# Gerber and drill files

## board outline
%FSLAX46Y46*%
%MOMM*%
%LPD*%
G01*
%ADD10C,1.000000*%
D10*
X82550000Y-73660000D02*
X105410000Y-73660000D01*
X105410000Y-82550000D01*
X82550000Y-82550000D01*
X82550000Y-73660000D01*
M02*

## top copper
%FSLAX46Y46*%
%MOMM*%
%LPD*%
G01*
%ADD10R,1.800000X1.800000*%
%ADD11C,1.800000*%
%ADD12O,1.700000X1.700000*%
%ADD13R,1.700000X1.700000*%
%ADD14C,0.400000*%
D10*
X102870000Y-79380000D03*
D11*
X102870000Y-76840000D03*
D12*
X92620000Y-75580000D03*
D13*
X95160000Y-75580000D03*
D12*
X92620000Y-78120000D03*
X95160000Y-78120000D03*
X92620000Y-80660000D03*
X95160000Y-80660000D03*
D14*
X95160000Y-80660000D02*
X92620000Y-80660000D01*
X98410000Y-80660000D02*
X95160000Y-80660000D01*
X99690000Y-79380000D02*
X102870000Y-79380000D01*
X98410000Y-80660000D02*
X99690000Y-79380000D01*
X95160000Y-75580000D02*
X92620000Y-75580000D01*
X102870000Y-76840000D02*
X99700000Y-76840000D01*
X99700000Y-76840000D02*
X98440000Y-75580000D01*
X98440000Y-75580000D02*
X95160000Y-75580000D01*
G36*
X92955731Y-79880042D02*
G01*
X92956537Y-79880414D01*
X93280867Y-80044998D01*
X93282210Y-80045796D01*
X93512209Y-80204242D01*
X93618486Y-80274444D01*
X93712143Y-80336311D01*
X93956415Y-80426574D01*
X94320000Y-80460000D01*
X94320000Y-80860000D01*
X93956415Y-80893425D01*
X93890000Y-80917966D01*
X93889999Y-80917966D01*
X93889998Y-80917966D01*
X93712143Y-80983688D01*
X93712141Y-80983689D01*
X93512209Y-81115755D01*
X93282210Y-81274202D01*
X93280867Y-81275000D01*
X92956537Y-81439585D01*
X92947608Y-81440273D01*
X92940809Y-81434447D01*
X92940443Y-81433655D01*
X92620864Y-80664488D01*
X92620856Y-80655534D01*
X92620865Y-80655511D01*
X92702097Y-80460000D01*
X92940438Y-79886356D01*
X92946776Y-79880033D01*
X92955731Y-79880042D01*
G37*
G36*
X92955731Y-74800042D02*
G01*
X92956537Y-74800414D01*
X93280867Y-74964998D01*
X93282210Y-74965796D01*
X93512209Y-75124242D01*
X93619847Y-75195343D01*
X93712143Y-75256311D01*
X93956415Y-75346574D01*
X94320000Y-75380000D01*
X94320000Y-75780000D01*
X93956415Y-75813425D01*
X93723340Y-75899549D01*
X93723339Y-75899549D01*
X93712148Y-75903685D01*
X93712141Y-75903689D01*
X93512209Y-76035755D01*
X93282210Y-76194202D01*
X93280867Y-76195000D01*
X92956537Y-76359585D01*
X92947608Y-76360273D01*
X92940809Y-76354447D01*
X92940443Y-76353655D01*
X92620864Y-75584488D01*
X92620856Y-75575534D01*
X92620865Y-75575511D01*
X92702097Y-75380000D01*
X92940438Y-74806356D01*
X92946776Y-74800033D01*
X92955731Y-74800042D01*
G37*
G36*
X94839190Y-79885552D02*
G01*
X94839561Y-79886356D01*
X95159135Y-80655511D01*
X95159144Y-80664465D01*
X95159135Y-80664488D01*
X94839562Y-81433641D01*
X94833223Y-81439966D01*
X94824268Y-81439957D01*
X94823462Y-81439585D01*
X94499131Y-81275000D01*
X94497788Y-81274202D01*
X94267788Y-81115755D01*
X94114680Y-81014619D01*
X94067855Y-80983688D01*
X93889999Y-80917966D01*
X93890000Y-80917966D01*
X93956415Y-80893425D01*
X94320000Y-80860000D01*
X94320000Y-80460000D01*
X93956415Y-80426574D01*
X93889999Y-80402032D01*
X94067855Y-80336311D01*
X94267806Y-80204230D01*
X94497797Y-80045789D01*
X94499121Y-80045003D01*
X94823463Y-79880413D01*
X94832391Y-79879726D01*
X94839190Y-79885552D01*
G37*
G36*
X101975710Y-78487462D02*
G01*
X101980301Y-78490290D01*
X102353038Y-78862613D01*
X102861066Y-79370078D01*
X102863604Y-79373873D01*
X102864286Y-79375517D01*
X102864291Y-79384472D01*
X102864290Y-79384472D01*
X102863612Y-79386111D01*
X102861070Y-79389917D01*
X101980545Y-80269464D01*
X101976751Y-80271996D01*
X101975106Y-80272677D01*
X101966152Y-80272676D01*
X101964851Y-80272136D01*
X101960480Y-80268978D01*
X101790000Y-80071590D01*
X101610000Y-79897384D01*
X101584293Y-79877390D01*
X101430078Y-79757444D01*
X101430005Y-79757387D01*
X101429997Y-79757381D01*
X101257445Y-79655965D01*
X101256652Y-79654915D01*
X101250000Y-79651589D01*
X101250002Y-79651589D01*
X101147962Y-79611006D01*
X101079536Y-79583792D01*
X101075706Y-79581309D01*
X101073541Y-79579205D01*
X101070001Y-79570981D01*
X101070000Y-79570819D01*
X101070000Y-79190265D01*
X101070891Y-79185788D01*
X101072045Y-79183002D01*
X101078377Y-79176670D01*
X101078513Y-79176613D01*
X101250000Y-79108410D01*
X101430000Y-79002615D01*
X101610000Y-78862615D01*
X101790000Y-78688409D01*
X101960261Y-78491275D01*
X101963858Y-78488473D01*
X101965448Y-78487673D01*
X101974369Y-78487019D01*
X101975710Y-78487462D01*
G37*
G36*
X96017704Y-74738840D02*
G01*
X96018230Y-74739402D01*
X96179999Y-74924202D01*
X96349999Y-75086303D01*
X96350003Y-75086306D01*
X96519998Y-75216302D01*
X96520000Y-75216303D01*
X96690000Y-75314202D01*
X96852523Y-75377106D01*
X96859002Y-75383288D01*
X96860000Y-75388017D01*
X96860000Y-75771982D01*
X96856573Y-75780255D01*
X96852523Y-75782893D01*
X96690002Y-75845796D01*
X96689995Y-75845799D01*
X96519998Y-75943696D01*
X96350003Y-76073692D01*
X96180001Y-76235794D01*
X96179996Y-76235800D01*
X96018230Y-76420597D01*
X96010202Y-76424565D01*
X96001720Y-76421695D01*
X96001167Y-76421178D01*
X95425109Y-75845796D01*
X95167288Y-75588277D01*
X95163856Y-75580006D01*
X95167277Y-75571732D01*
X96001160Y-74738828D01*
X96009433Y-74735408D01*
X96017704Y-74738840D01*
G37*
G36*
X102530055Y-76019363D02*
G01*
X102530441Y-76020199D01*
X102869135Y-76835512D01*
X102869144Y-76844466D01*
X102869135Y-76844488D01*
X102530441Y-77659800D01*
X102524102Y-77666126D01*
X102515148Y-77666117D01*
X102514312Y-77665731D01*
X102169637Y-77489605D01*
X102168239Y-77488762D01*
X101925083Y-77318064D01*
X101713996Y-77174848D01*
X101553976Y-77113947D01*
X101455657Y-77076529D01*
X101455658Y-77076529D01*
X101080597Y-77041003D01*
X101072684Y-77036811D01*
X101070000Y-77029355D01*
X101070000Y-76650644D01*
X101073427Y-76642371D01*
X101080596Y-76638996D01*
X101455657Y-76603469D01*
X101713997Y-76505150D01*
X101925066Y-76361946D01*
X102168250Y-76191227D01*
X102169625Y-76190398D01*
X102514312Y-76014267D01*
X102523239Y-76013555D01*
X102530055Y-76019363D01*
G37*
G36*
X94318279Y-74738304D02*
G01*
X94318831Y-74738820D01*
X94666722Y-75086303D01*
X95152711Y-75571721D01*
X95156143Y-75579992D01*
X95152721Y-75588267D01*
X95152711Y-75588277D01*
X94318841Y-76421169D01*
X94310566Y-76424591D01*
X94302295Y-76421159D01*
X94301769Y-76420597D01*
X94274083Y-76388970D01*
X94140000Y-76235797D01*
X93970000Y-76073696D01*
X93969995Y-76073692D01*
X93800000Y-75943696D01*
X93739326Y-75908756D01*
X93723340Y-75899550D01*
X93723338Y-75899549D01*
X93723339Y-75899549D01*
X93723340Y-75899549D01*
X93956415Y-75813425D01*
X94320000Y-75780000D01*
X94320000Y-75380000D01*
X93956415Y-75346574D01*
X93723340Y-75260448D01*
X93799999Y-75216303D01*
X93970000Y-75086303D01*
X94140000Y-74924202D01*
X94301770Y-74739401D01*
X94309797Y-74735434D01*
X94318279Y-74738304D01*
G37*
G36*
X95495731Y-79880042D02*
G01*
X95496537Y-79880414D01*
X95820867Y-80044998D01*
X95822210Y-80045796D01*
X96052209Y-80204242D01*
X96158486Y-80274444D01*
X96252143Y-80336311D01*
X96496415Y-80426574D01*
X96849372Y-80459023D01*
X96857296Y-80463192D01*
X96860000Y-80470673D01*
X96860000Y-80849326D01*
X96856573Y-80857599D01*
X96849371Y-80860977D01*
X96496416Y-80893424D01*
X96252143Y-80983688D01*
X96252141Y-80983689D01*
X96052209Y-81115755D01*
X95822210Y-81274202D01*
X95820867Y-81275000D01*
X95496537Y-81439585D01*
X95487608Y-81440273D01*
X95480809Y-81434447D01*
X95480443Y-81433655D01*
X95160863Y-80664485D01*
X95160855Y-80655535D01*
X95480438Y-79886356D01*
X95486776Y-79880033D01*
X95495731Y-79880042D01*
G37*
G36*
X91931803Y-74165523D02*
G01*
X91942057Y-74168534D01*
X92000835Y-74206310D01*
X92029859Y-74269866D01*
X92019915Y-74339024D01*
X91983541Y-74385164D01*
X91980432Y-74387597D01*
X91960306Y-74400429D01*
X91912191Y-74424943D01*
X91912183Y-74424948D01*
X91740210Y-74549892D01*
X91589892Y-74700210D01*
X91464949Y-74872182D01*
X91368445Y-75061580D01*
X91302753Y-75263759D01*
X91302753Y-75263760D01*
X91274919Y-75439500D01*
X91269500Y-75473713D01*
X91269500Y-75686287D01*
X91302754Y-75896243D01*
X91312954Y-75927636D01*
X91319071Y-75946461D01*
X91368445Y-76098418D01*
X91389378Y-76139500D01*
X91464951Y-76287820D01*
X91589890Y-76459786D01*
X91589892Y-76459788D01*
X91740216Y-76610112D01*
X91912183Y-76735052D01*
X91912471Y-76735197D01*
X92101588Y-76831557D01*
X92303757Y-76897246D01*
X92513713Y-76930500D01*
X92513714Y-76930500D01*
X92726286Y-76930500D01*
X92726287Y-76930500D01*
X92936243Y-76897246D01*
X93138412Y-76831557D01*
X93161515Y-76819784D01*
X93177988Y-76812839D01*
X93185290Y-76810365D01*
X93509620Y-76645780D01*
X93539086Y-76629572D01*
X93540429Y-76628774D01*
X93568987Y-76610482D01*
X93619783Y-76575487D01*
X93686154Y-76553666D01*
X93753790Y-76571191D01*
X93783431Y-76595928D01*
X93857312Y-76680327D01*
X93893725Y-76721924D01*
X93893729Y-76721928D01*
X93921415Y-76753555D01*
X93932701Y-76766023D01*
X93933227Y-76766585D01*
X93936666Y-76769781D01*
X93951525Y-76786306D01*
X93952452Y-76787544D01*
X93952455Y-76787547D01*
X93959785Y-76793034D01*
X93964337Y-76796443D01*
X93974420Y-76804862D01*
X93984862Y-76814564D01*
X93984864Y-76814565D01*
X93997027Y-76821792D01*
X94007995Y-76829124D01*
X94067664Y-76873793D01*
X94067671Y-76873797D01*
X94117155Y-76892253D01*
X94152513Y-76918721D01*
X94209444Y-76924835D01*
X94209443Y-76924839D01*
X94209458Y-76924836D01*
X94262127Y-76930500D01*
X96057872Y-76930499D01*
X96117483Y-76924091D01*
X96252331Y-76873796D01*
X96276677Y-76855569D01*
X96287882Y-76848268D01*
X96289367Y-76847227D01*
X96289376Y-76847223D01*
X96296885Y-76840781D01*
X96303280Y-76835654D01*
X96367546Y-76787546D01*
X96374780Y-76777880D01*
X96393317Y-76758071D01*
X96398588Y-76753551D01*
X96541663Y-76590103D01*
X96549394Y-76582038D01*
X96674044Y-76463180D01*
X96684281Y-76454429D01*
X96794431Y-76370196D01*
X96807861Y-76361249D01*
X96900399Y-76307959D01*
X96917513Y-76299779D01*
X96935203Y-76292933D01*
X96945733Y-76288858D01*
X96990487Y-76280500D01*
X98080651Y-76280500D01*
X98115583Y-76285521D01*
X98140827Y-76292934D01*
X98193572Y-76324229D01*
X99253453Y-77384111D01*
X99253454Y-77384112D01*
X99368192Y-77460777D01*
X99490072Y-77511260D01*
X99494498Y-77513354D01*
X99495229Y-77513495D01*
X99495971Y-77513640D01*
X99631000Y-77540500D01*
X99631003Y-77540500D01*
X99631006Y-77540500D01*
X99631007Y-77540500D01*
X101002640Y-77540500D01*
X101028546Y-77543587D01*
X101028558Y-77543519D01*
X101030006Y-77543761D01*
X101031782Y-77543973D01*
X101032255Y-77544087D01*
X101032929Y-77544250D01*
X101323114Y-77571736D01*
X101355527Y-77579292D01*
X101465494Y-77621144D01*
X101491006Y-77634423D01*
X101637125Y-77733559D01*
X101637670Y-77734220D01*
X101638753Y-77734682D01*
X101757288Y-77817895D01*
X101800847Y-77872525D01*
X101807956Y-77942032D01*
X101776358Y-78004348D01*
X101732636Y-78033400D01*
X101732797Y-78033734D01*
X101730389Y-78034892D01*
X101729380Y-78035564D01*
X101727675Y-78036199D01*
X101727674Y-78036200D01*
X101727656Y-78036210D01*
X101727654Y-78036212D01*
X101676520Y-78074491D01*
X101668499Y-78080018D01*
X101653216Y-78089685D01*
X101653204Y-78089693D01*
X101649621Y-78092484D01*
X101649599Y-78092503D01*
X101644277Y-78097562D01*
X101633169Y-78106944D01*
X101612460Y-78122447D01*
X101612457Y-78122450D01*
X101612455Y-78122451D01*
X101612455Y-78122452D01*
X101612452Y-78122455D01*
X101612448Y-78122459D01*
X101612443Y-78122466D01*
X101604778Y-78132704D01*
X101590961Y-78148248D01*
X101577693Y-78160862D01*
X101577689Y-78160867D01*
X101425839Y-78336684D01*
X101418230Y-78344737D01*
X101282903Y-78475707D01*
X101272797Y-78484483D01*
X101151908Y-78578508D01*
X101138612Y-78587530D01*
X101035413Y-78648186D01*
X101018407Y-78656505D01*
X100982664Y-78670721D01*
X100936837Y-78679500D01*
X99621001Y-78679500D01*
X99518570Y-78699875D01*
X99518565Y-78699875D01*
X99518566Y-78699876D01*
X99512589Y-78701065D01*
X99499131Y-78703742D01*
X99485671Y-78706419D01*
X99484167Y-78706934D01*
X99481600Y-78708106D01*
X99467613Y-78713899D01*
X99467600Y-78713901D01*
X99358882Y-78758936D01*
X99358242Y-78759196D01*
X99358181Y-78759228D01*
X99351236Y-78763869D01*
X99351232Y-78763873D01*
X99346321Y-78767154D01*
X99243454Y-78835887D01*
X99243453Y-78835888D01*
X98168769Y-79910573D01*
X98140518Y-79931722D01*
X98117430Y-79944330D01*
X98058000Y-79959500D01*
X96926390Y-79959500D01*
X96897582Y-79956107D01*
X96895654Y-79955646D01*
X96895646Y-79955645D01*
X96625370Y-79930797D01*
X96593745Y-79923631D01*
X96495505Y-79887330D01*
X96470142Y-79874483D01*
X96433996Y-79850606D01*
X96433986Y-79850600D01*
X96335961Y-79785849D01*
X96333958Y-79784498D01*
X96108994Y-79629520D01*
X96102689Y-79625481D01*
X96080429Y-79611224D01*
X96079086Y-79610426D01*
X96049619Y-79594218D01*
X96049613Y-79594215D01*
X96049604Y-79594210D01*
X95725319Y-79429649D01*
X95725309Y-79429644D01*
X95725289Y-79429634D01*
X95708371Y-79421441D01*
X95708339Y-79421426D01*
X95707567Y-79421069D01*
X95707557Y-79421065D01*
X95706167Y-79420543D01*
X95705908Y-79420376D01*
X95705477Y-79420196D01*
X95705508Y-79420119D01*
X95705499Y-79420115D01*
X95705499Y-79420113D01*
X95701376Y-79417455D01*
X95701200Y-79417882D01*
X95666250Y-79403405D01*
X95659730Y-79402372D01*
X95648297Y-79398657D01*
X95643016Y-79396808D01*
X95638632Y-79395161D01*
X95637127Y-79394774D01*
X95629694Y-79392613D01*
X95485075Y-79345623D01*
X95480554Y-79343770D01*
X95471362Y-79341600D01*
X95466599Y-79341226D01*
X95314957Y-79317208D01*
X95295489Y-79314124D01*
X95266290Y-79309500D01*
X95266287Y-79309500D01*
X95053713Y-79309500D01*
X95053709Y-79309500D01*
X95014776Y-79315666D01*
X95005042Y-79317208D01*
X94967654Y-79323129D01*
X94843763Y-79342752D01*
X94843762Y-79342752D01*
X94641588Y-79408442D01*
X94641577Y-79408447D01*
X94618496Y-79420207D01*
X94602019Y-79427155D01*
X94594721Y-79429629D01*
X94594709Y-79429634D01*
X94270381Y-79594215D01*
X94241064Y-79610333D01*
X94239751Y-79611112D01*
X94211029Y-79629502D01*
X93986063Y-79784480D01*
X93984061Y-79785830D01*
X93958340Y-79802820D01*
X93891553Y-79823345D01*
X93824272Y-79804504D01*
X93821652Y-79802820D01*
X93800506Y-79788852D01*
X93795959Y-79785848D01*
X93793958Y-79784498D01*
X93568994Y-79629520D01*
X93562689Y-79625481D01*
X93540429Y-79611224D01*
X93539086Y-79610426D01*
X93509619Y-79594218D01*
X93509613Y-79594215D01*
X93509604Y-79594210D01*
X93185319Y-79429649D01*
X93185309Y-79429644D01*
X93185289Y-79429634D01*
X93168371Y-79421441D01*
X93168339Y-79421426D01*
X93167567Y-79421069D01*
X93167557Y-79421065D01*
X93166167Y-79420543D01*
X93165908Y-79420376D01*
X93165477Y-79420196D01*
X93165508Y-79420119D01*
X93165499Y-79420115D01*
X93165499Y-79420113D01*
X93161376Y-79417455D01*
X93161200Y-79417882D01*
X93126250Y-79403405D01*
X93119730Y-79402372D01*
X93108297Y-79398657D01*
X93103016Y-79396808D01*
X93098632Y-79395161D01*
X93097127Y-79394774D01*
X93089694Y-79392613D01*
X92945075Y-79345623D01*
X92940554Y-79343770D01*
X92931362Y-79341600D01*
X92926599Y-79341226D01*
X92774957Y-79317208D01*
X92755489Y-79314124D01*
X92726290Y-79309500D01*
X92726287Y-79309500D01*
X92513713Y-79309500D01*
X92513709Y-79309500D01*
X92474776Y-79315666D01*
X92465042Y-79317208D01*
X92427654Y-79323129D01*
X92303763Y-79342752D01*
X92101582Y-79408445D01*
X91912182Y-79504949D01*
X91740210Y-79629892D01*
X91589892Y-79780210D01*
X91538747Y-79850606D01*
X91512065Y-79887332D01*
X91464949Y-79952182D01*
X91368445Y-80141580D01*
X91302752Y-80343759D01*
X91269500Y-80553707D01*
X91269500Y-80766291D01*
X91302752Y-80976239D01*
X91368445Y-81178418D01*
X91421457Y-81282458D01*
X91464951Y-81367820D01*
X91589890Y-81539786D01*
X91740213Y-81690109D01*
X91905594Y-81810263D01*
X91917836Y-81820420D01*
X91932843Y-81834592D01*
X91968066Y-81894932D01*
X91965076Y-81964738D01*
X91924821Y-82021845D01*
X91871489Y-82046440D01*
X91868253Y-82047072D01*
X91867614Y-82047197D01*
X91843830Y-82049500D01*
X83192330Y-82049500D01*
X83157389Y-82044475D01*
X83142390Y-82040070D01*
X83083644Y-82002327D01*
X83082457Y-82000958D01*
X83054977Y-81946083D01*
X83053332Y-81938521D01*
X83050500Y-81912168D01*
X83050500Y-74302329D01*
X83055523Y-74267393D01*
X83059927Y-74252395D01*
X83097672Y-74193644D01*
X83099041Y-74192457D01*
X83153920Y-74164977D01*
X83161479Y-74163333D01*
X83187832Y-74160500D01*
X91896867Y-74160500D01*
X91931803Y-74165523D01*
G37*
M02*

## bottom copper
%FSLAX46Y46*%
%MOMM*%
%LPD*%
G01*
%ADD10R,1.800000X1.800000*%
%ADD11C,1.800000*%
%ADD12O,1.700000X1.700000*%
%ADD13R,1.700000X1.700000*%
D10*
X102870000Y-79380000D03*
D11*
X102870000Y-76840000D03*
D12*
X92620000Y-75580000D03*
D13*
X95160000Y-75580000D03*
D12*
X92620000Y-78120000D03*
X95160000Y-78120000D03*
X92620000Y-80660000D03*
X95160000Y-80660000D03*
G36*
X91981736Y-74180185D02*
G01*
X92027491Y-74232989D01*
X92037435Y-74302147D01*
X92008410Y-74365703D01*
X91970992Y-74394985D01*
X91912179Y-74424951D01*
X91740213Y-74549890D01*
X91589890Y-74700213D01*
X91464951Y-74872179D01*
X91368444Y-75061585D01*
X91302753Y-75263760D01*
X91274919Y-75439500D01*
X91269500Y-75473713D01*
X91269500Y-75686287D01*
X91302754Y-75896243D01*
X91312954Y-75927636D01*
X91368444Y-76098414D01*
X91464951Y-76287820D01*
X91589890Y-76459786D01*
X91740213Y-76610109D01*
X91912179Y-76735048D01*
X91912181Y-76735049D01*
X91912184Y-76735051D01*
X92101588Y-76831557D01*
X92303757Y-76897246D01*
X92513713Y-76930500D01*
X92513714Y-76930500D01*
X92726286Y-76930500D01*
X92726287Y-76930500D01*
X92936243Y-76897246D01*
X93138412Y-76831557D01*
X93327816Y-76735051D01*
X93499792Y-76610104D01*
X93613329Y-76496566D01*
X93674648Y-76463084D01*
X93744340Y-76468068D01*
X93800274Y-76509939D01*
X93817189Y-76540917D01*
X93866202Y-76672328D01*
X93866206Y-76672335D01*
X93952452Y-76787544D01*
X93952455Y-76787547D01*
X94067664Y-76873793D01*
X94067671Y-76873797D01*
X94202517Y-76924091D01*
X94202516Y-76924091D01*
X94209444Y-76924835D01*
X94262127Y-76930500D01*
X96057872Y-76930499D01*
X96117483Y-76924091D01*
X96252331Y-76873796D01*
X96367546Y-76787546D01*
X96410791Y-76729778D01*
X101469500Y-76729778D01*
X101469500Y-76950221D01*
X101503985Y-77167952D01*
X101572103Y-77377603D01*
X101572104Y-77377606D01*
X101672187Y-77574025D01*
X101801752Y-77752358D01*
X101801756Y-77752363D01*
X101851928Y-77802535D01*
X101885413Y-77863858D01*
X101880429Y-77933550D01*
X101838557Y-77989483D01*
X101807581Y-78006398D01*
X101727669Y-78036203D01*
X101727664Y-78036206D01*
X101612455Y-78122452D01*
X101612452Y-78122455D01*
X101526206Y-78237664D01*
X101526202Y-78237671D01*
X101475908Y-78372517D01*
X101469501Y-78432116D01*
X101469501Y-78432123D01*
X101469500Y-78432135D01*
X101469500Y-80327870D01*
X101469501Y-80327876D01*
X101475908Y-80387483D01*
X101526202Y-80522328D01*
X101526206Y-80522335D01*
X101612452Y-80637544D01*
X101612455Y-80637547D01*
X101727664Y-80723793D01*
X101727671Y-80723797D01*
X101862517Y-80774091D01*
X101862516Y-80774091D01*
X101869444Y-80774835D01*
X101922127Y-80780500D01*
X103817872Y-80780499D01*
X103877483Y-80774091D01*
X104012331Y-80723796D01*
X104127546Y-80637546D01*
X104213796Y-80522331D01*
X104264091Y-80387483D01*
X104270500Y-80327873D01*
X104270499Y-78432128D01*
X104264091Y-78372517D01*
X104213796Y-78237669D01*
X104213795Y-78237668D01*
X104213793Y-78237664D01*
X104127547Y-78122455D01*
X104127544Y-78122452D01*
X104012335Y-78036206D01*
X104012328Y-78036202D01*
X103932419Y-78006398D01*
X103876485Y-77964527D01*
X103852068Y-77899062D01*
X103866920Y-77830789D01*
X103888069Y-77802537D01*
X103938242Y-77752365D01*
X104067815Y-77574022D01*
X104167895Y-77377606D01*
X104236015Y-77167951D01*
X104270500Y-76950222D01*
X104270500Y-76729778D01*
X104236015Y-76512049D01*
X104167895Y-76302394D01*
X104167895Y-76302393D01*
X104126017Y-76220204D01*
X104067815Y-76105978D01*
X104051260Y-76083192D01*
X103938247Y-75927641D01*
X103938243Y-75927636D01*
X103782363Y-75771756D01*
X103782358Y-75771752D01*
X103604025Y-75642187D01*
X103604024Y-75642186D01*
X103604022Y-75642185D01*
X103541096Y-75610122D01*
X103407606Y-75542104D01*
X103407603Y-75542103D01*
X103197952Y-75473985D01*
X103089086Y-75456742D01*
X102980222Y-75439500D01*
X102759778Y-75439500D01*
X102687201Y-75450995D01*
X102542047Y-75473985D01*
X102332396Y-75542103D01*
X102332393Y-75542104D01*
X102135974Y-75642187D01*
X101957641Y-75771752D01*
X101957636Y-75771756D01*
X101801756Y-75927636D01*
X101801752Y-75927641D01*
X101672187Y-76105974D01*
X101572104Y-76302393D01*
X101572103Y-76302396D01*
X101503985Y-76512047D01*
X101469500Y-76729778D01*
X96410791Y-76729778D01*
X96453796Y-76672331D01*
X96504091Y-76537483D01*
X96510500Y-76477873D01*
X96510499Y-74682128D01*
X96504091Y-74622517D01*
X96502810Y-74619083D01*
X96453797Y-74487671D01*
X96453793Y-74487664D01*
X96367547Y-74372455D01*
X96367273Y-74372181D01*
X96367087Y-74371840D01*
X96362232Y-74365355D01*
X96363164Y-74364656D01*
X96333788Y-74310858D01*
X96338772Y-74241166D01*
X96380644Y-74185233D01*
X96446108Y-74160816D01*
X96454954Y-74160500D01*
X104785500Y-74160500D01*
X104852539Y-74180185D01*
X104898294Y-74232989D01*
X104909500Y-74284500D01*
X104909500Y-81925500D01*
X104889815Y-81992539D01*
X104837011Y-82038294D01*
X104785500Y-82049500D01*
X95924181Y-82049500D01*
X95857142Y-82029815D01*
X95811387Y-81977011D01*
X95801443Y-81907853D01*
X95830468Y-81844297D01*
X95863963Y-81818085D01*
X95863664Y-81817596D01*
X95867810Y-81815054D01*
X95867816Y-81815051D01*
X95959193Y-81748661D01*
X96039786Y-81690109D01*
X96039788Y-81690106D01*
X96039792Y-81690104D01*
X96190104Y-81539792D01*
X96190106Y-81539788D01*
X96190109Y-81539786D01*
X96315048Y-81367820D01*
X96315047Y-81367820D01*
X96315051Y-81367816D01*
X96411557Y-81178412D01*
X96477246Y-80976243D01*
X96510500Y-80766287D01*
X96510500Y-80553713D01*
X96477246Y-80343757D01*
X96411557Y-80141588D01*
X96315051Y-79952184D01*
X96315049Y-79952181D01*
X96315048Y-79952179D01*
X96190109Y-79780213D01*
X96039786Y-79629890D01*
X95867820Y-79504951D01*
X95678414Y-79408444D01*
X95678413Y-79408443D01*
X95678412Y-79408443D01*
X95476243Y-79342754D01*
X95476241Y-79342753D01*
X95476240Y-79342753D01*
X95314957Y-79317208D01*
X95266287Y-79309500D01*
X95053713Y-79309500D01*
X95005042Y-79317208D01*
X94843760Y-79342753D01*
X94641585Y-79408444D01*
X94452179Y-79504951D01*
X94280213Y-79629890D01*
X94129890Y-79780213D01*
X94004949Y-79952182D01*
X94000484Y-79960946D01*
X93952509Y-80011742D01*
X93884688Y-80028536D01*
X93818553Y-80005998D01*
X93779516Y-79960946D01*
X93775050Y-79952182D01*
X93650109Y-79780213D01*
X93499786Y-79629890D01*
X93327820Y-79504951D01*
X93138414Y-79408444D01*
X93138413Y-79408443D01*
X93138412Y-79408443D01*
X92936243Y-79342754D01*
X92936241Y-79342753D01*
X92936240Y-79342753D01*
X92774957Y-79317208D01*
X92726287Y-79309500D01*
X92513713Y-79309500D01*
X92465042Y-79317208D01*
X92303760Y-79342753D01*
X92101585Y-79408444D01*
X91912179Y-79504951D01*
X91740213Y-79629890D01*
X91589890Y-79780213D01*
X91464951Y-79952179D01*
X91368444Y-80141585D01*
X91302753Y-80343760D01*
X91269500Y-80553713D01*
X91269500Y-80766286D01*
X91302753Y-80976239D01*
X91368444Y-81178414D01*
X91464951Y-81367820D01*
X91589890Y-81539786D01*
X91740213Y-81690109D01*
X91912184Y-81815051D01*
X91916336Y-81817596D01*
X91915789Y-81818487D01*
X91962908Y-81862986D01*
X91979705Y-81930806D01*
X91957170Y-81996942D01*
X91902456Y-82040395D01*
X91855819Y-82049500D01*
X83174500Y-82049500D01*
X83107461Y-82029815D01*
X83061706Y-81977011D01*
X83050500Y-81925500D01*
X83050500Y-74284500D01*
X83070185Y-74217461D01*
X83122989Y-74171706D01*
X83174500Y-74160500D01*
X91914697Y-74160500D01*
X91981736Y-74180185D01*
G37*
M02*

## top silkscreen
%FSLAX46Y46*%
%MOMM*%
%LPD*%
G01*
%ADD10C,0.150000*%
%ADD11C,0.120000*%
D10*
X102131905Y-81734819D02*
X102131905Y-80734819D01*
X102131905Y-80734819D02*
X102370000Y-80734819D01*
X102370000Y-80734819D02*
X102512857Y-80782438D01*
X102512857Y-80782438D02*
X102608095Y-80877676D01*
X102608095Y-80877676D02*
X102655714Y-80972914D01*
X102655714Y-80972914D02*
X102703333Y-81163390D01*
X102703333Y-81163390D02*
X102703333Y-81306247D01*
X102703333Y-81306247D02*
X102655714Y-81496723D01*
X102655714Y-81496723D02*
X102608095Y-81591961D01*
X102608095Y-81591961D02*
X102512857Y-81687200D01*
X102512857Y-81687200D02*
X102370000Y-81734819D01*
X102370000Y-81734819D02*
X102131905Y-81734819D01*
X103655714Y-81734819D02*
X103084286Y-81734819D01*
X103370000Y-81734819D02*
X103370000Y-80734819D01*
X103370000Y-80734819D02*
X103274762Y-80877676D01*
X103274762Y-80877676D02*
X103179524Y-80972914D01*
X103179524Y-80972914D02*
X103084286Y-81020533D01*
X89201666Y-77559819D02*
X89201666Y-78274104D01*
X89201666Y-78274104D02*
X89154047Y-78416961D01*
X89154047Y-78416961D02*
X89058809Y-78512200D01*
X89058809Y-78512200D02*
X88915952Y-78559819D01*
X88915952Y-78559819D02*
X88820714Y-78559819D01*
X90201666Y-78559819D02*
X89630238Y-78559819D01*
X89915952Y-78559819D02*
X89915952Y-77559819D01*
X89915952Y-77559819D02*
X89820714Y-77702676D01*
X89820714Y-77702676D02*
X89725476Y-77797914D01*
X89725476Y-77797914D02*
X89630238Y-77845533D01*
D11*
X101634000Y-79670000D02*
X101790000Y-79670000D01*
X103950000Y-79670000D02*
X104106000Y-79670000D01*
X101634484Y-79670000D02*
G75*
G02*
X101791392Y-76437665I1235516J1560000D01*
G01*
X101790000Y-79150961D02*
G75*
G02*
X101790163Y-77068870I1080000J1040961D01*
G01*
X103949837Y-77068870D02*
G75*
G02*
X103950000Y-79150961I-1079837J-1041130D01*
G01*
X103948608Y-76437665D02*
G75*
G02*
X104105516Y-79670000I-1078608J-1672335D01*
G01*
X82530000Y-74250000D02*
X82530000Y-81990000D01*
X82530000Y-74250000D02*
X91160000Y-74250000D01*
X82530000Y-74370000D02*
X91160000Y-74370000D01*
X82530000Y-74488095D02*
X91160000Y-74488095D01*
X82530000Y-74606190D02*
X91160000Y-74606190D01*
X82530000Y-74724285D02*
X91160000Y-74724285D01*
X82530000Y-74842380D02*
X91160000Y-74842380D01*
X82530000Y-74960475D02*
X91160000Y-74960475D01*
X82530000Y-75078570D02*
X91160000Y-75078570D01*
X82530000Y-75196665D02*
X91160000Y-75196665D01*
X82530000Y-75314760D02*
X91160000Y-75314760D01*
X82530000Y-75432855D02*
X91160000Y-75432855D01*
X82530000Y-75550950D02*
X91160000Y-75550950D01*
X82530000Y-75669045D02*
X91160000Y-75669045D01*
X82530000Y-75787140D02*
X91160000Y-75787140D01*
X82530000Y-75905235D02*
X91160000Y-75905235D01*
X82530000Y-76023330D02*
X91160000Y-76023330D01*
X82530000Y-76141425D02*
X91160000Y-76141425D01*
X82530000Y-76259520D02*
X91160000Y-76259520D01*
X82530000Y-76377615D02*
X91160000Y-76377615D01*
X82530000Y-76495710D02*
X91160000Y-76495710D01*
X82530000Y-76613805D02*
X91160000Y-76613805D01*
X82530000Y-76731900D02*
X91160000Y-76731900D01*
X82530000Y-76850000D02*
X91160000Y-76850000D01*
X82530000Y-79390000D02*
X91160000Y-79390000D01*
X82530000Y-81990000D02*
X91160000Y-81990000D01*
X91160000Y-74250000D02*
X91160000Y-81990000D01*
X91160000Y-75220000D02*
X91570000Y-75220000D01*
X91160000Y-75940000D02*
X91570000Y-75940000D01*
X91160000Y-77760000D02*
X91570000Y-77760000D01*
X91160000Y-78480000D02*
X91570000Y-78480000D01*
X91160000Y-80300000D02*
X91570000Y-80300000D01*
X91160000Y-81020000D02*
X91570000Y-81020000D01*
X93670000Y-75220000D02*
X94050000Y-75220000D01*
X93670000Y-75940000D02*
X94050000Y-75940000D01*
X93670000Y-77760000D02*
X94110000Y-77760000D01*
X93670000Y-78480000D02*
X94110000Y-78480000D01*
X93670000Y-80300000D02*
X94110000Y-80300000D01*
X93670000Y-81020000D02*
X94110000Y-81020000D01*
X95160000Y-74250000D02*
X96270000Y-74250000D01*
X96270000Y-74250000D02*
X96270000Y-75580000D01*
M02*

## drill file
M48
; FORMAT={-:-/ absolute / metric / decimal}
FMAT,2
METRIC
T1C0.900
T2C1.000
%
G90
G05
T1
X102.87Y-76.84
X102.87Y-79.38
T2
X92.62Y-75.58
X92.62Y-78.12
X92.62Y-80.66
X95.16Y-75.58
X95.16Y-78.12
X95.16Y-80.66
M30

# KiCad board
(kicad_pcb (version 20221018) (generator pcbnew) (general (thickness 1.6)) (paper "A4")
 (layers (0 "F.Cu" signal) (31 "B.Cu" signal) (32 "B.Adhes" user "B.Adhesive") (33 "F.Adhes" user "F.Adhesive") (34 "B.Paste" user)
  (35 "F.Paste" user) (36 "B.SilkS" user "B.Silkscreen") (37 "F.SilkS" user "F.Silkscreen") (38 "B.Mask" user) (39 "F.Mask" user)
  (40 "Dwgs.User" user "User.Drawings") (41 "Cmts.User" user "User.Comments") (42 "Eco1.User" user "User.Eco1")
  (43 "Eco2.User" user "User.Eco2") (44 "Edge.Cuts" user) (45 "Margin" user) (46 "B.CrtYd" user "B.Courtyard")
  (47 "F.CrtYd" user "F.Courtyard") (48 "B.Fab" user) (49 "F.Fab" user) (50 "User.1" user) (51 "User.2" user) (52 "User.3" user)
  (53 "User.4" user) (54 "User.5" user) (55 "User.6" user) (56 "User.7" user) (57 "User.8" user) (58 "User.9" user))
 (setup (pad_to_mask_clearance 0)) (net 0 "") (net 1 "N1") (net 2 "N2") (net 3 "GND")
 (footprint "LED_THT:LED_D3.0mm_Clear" (layer "F.Cu") (at 102.87 79.38 90)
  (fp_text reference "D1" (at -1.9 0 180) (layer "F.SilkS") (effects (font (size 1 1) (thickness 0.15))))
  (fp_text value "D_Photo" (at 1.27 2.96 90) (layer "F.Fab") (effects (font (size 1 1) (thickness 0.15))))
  (fp_line (start -0.29 -1.236) (end -0.29 -1.08) (stroke (width 0.12) (type solid)) (layer "F.SilkS"))
  (fp_line (start -0.29 1.08) (end -0.29 1.236) (stroke (width 0.12) (type solid)) (layer "F.SilkS"))
  (fp_arc (start -0.29 -1.235516) (mid 1.366487 -1.987659) (end 2.942335 -1.078608) (stroke (width 0.12) (type solid)) (layer "F.SilkS"))
  (fp_arc (start 0.229039 -1.08) (mid 1.270117 -1.5) (end 2.31113 -1.079837) (stroke (width 0.12) (type solid)) (layer "F.SilkS"))
  (fp_arc (start 2.31113 1.079837) (mid 1.270117 1.5) (end 0.229039 1.08) (stroke (width 0.12) (type solid)) (layer "F.SilkS"))
  (fp_arc (start 2.942335 1.078608) (mid 1.366487 1.987659) (end -0.29 1.235516) (stroke (width 0.12) (type solid)) (layer "F.SilkS"))
  (pad "1" thru_hole rect (at 0 0 90) (size 1.8 1.8) (drill 0.9) (layers "*.Cu" "*.Mask") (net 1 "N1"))
  (pad "2" thru_hole circle (at 2.54 0 90) (size 1.8 1.8) (drill 0.9) (layers "*.Cu" "*.Mask") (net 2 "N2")))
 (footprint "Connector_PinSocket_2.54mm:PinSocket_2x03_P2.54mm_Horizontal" (layer "F.Cu") (at 95.16 75.58)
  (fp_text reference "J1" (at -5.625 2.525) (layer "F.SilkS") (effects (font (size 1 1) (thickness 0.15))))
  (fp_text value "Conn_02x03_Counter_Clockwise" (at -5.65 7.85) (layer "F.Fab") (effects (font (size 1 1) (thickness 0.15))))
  (fp_line (start -12.63 -1.33) (end -12.63 6.41) (stroke (width 0.12) (type solid)) (layer "F.SilkS"))
  (fp_line (start -12.63 -1.33) (end -4 -1.33) (stroke (width 0.12) (type solid)) (layer "F.SilkS"))
  (fp_line (start -12.63 -1.21) (end -4 -1.21) (stroke (width 0.12) (type solid)) (layer "F.SilkS"))
  (fp_line (start -12.63 -1.091905) (end -4 -1.091905) (stroke (width 0.12) (type solid)) (layer "F.SilkS"))
  (fp_line (start -12.63 -0.97381) (end -4 -0.97381) (stroke (width 0.12) (type solid)) (layer "F.SilkS"))
  (fp_line (start -12.63 -0.855715) (end -4 -0.855715) (stroke (width 0.12) (type solid)) (layer "F.SilkS"))
  (fp_line (start -12.63 -0.73762) (end -4 -0.73762) (stroke (width 0.12) (type solid)) (layer "F.SilkS"))
  (fp_line (start -12.63 -0.619525) (end -4 -0.619525) (stroke (width 0.12) (type solid)) (layer "F.SilkS"))
  (fp_line (start -12.63 -0.50143) (end -4 -0.50143) (stroke (width 0.12) (type solid)) (layer "F.SilkS"))
  (fp_line (start -12.63 -0.383335) (end -4 -0.383335) (stroke (width 0.12) (type solid)) (layer "F.SilkS"))
  (fp_line (start -12.63 -0.26524) (end -4 -0.26524) (stroke (width 0.12) (type solid)) (layer "F.SilkS"))
  (fp_line (start -12.63 -0.147145) (end -4 -0.147145) (stroke (width 0.12) (type solid)) (layer "F.SilkS"))
  (fp_line (start -12.63 -0.02905) (end -4 -0.02905) (stroke (width 0.12) (type solid)) (layer "F.SilkS"))
  (fp_line (start -12.63 0.089045) (end -4 0.089045) (stroke (width 0.12) (type solid)) (layer "F.SilkS"))
  (fp_line (start -12.63 0.20714) (end -4 0.20714) (stroke (width 0.12) (type solid)) (layer "F.SilkS"))
  (fp_line (start -12.63 0.325235) (end -4 0.325235) (stroke (width 0.12) (type solid)) (layer "F.SilkS"))
  (fp_line (start -12.63 0.44333) (end -4 0.44333) (stroke (width 0.12) (type solid)) (layer "F.SilkS"))
  (fp_line (start -12.63 0.561425) (end -4 0.561425) (stroke (width 0.12) (type solid)) (layer "F.SilkS"))
  (fp_line (start -12.63 0.67952) (end -4 0.67952) (stroke (width 0.12) (type solid)) (layer "F.SilkS"))
  (fp_line (start -12.63 0.797615) (end -4 0.797615) (stroke (width 0.12) (type solid)) (layer "F.SilkS"))
  (fp_line (start -12.63 0.91571) (end -4 0.91571) (stroke (width 0.12) (type solid)) (layer "F.SilkS"))
  (fp_line (start -12.63 1.033805) (end -4 1.033805) (stroke (width 0.12) (type solid)) (layer "F.SilkS"))
  (fp_line (start -12.63 1.1519) (end -4 1.1519) (stroke (width 0.12) (type solid)) (layer "F.SilkS"))
  (fp_line (start -12.63 1.27) (end -4 1.27) (stroke (width 0.12) (type solid)) (layer "F.SilkS"))
  (fp_line (start -12.63 3.81) (end -4 3.81) (stroke (width 0.12) (type solid)) (layer "F.SilkS"))
  (fp_line (start -12.63 6.41) (end -4 6.41) (stroke (width 0.12) (type solid)) (layer "F.SilkS"))
  (fp_line (start -4 -1.33) (end -4 6.41) (stroke (width 0.12) (type solid)) (layer "F.SilkS"))
  (fp_line (start -4 -0.36) (end -3.59 -0.36) (stroke (width 0.12) (type solid)) (layer "F.SilkS"))
  (fp_line (start -4 0.36) (end -3.59 0.36) (stroke (width 0.12) (type solid)) (layer "F.SilkS"))
  (fp_line (start -4 2.18) (end -3.59 2.18) (stroke (width 0.12) (type solid)) (layer "F.SilkS"))
  (fp_line (start -4 2.9) (end -3.59 2.9) (stroke (width 0.12) (type solid)) (layer "F.SilkS"))
  (fp_line (start -4 4.72) (end -3.59 4.72) (stroke (width 0.12) (type solid)) (layer "F.SilkS"))
  (fp_line (start -4 5.44) (end -3.59 5.44) (stroke (width 0.12) (type solid)) (layer "F.SilkS"))
  (fp_line (start -1.49 -0.36) (end -1.11 -0.36) (stroke (width 0.12) (type solid)) (layer "F.SilkS"))
  (fp_line (start -1.49 0.36) (end -1.11 0.36) (stroke (width 0.12) (type solid)) (layer "F.SilkS"))
  (fp_line (start -1.49 2.18) (end -1.05 2.18) (stroke (width 0.12) (type solid)) (layer "F.SilkS"))
  (fp_line (start -1.49 2.9) (end -1.05 2.9) (stroke (width 0.12) (type solid)) (layer "F.SilkS"))
  (fp_line (start -1.49 4.72) (end -1.05 4.72) (stroke (width 0.12) (type solid)) (layer "F.SilkS"))
  (fp_line (start -1.49 5.44) (end -1.05 5.44) (stroke (width 0.12) (type solid)) (layer "F.SilkS"))
  (fp_line (start 0 -1.33) (end 1.11 -1.33) (stroke (width 0.12) (type solid)) (layer "F.SilkS"))
  (fp_line (start 1.11 -1.33) (end 1.11 0) (stroke (width 0.12) (type solid)) (layer "F.SilkS"))
  (pad "1" thru_hole oval (at -2.54 0) (size 1.7 1.7) (drill 1) (layers "*.Cu" "*.Mask") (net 2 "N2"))
  (pad "1" thru_hole rect (at 0 0) (size 1.7 1.7) (drill 1) (layers "*.Cu" "*.Mask") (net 2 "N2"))
  (pad "2" thru_hole oval (at -2.54 2.54) (size 1.7 1.7) (drill 1) (layers "*.Cu" "*.Mask") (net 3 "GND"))
  (pad "2" thru_hole oval (at 0 2.54) (size 1.7 1.7) (drill 1) (layers "*.Cu" "*.Mask") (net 3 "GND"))
  (pad "3" thru_hole oval (at -2.54 5.08) (size 1.7 1.7) (drill 1) (layers "*.Cu" "*.Mask") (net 1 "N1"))
  (pad "3" thru_hole oval (at 0 5.08) (size 1.7 1.7) (drill 1) (layers "*.Cu" "*.Mask") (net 1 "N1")))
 (gr_rect (start 82.55 73.66) (end 105.41 82.55) (stroke (width 1) (type default)) (fill none) (layer "Edge.Cuts"))
 (segment (start 95.16 80.66) (end 92.62 80.66) (width 0.4) (layer "F.Cu") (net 1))
 (segment (start 98.41 80.66) (end 95.16 80.66) (width 0.4) (layer "F.Cu") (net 1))
 (segment (start 99.69 79.38) (end 102.87 79.38) (width 0.4) (layer "F.Cu") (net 1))
 (segment (start 98.41 80.66) (end 99.69 79.38) (width 0.4) (layer "F.Cu") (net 1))
 (segment (start 95.16 75.58) (end 92.62 75.58) (width 0.4) (layer "F.Cu") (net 2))
 (segment (start 102.87 76.84) (end 99.7 76.84) (width 0.4) (layer "F.Cu") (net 2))
 (segment (start 99.7 76.84) (end 98.44 75.58) (width 0.4) (layer "F.Cu") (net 2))
 (segment (start 98.44 75.58) (end 95.16 75.58) (width 0.4) (layer "F.Cu") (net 2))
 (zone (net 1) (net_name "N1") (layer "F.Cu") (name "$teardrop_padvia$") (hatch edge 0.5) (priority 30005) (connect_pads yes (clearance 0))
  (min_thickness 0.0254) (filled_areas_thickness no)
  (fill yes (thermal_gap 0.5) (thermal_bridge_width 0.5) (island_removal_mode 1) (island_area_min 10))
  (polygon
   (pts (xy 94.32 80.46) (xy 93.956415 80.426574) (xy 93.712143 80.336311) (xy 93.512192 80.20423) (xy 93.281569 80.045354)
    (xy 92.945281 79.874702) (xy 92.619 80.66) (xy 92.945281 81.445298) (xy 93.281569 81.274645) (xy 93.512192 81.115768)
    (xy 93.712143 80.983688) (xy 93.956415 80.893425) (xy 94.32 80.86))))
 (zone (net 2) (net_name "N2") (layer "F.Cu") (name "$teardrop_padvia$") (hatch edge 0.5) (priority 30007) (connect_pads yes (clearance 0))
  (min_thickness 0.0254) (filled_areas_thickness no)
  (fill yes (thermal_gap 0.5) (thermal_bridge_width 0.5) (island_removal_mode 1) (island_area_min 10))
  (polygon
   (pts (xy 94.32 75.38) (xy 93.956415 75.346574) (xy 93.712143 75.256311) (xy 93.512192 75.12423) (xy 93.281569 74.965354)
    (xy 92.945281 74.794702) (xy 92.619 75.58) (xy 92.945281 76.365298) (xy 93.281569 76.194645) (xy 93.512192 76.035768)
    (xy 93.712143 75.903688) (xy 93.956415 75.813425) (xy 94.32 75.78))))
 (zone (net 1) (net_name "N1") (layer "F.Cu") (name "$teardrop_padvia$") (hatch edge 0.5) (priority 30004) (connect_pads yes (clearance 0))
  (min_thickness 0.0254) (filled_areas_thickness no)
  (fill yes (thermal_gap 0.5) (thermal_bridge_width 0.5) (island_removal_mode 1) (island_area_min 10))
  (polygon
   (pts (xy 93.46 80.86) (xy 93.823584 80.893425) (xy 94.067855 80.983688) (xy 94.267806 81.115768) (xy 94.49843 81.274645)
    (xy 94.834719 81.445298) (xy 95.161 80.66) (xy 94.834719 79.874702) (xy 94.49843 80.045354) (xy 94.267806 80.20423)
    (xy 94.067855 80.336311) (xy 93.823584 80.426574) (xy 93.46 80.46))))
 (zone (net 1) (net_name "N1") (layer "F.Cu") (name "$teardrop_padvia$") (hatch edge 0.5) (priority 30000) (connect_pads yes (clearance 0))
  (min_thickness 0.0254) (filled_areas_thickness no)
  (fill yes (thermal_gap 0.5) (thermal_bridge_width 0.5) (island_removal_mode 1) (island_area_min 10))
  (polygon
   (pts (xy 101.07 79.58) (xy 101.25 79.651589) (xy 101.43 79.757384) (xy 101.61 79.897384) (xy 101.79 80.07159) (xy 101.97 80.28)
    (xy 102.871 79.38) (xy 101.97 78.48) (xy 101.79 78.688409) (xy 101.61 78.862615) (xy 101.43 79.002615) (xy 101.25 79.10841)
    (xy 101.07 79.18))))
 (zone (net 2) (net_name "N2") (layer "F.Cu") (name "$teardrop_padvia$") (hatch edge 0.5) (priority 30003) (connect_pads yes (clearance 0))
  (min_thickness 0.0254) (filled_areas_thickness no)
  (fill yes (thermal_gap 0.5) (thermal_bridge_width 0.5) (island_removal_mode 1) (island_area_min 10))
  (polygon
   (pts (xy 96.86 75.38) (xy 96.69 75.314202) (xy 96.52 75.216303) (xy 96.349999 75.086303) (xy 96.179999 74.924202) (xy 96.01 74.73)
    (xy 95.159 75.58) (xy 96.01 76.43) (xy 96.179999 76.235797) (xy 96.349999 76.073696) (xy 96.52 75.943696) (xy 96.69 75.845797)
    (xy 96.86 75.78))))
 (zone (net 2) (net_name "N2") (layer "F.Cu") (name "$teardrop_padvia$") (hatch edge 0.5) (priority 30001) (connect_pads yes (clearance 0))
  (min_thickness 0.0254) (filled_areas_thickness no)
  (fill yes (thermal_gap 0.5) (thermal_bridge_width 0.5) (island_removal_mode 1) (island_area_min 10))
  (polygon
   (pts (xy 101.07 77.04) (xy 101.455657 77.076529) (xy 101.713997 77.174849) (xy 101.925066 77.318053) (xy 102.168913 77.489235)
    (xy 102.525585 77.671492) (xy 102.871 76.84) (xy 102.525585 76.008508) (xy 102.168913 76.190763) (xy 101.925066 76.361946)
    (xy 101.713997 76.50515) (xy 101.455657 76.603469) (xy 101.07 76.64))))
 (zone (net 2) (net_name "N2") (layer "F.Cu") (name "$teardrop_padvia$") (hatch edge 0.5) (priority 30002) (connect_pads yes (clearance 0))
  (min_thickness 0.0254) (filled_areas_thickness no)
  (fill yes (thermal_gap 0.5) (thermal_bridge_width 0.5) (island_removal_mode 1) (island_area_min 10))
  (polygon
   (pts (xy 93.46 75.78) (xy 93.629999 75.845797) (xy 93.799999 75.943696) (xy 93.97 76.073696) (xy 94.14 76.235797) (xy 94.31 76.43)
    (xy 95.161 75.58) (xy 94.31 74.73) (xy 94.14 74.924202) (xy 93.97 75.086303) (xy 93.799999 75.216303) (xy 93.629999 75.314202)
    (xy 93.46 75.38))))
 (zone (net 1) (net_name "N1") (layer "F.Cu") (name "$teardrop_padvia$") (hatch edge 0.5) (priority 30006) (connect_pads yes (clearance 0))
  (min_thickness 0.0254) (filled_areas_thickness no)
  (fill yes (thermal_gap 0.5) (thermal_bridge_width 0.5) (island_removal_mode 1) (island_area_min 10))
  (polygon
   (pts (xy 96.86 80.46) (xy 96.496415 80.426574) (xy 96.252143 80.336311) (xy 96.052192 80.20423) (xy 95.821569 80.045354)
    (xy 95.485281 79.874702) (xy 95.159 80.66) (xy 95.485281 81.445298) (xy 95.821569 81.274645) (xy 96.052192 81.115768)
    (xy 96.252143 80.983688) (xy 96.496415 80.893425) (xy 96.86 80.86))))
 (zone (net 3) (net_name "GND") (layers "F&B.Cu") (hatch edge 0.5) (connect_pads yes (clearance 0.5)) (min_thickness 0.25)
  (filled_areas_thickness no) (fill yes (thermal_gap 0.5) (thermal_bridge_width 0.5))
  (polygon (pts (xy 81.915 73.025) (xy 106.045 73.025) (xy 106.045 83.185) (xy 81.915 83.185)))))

